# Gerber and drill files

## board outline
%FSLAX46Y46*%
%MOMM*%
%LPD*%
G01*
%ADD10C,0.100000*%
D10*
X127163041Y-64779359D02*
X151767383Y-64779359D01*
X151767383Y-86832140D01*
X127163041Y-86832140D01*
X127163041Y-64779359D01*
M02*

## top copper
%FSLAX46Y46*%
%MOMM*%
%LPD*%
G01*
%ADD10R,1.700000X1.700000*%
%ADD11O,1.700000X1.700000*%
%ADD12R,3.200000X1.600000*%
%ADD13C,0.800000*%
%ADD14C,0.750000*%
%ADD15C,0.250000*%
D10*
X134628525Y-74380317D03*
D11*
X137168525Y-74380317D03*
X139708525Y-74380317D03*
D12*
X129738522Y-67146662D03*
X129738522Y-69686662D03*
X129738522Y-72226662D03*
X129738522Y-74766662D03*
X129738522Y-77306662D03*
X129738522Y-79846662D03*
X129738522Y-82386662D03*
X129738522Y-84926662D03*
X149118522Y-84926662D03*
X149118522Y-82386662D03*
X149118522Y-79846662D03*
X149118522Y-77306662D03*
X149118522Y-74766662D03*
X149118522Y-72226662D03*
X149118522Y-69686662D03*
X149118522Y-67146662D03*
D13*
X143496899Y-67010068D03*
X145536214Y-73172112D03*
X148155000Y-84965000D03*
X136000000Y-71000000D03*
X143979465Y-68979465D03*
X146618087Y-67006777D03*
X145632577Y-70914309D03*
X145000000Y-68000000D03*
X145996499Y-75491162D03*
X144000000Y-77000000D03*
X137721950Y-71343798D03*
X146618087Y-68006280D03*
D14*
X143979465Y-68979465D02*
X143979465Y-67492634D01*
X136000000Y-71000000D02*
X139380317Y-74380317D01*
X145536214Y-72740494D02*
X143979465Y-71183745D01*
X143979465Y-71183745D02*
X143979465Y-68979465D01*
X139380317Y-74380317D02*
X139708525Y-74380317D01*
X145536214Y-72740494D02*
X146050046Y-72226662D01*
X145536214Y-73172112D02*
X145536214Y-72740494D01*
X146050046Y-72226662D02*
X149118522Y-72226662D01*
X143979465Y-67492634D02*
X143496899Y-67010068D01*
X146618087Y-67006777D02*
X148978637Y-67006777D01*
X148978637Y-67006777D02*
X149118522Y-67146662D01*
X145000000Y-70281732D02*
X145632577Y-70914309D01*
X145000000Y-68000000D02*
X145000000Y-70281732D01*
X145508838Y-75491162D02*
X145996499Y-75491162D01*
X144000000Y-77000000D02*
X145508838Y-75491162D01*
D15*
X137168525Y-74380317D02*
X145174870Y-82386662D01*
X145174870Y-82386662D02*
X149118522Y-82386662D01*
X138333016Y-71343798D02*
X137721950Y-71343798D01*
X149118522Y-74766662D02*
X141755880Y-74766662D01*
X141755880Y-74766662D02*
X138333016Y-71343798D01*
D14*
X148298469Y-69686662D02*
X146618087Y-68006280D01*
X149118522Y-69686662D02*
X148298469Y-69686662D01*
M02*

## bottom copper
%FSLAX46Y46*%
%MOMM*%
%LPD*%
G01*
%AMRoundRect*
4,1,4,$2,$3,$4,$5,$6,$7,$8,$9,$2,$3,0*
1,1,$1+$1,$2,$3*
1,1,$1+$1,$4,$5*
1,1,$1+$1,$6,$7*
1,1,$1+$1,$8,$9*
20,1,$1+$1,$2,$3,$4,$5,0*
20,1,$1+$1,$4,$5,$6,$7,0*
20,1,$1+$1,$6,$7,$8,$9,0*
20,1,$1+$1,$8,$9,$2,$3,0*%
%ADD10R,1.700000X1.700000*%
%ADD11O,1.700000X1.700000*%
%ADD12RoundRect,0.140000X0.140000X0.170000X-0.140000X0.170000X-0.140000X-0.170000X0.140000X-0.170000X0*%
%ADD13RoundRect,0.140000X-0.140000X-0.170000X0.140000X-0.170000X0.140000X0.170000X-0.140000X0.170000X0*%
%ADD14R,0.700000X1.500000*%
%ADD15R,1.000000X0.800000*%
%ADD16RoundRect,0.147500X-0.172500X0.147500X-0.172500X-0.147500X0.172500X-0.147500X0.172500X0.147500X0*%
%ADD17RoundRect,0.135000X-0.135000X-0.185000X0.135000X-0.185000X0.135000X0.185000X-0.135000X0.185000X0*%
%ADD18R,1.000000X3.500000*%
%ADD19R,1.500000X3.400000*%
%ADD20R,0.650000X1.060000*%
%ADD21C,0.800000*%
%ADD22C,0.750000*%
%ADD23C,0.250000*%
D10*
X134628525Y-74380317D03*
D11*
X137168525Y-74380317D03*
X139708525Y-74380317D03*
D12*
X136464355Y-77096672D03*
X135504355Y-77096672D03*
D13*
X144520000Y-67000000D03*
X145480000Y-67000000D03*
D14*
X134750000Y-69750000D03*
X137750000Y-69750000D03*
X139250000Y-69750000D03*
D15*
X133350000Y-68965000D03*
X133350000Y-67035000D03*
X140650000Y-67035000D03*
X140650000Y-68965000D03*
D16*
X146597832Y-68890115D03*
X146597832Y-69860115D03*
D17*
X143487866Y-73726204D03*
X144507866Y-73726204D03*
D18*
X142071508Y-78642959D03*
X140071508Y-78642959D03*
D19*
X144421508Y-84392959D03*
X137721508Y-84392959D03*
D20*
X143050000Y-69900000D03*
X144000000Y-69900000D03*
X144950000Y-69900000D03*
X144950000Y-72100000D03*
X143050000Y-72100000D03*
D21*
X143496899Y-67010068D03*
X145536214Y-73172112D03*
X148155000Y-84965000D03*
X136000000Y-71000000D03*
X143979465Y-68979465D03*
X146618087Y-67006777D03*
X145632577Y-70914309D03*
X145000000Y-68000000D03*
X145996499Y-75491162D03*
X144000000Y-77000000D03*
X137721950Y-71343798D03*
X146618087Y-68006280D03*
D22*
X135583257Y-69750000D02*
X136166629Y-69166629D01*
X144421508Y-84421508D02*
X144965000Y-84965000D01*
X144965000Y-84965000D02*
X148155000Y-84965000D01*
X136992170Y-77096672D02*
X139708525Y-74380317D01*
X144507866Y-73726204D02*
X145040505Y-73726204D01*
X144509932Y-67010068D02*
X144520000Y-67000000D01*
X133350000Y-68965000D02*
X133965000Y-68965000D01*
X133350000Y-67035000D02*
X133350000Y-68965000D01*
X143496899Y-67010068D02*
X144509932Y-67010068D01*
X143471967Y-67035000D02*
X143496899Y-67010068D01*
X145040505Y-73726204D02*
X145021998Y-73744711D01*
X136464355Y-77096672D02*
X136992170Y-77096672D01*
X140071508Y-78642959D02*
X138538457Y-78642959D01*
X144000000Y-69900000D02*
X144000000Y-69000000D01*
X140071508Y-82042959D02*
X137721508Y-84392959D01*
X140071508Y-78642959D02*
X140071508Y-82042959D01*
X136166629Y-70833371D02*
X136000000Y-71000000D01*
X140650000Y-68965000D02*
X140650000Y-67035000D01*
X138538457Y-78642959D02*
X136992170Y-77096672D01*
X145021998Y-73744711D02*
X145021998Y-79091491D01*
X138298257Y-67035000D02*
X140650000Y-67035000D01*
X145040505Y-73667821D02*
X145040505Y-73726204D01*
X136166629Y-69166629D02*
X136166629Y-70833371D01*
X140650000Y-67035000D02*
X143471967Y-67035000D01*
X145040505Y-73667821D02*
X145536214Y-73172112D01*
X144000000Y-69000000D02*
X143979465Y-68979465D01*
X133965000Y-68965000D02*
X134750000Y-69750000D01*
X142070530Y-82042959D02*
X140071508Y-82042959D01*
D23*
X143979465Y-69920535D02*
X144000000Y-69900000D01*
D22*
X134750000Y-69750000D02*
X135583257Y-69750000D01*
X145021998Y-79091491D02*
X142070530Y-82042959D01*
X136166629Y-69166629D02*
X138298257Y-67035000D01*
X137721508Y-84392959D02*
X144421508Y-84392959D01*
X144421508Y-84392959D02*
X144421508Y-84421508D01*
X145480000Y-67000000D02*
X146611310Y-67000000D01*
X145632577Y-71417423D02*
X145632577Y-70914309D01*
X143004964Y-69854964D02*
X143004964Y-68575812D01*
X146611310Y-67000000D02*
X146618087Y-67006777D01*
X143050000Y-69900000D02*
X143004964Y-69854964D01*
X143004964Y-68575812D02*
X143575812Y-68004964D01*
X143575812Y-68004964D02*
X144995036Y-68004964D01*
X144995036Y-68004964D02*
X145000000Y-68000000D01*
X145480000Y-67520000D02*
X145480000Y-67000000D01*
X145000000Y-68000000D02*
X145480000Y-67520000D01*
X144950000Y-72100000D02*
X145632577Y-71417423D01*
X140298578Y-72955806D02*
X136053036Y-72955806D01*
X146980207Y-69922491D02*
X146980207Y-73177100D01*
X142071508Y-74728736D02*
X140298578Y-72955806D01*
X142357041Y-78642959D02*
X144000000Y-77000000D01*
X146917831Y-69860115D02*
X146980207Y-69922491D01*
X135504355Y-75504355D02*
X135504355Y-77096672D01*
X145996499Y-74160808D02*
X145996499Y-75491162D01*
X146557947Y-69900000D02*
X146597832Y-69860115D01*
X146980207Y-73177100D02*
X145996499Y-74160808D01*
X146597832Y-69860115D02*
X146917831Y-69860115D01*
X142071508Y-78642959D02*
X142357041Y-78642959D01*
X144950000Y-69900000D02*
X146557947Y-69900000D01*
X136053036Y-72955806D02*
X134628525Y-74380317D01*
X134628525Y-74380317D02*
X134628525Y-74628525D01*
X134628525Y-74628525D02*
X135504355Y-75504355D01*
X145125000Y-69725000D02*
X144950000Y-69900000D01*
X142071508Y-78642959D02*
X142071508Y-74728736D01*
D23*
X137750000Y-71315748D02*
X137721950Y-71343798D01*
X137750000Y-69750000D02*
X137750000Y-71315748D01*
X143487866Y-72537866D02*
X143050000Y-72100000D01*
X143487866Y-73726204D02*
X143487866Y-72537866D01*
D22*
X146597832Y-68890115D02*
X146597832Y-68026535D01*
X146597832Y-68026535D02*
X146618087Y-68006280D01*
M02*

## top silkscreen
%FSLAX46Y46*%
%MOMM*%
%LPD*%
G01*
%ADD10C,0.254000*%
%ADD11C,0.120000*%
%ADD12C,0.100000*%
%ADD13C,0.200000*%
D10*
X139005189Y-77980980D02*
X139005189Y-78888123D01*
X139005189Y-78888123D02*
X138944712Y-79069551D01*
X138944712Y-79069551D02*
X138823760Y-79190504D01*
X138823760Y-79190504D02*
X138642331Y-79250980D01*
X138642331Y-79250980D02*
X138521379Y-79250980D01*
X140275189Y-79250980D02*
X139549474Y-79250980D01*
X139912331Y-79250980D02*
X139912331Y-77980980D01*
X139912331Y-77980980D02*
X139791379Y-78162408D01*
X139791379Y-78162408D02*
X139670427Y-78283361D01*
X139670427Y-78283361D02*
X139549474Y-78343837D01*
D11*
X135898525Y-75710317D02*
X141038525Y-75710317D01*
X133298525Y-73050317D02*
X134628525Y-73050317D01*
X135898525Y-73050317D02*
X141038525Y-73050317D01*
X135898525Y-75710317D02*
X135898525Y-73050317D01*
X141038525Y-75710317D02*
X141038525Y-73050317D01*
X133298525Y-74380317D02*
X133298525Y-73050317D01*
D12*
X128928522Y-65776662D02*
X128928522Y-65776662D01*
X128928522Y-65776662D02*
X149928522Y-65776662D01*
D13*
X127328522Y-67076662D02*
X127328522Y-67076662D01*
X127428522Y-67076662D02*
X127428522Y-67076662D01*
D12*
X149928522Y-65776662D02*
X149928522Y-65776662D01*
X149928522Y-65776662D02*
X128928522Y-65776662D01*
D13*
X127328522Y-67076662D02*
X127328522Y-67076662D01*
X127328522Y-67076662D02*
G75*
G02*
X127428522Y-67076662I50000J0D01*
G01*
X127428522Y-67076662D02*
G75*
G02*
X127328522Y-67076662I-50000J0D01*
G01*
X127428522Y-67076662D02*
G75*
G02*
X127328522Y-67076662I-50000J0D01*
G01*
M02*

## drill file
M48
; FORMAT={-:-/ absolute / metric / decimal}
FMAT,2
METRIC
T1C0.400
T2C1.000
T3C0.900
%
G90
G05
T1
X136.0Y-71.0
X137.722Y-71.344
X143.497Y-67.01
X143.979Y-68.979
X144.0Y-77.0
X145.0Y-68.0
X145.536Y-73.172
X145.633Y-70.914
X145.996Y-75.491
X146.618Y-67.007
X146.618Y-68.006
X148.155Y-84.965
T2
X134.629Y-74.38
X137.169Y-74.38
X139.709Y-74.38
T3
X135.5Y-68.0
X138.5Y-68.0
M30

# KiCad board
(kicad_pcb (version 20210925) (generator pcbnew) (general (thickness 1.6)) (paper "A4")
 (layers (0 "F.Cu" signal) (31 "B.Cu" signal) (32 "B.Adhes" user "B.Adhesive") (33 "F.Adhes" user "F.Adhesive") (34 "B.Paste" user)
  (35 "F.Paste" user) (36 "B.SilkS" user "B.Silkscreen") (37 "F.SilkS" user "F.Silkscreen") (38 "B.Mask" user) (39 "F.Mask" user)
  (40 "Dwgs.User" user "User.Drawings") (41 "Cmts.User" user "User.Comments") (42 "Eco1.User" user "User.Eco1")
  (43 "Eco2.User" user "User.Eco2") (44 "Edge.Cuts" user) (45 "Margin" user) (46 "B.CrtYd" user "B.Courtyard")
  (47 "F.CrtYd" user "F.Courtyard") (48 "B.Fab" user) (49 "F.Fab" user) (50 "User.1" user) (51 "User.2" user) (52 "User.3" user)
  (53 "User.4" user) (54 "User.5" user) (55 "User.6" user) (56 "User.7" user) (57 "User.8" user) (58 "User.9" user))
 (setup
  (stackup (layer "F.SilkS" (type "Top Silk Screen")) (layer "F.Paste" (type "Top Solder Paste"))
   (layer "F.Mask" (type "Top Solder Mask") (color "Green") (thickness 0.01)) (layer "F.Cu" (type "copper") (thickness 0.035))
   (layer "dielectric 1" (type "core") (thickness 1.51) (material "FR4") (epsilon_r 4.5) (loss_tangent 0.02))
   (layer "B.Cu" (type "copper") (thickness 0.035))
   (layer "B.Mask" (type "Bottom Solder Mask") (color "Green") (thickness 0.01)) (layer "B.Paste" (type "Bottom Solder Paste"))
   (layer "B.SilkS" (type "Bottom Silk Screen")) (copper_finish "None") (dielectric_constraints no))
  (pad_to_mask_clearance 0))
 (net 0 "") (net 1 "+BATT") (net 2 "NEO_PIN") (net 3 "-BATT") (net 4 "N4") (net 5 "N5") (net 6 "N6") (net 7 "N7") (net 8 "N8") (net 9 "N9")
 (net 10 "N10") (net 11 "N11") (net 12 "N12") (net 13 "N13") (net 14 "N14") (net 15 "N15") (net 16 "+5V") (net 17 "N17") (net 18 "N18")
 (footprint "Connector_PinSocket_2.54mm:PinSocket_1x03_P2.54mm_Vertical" (layer "F.Cu") (at 134.628525 74.380317 90)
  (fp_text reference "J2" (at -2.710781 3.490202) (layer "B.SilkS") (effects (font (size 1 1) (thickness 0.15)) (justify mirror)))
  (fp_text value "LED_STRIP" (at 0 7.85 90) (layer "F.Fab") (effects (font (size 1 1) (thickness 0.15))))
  (fp_line (start -1.33 1.27) (end -1.33 6.41) (layer "F.SilkS") (width 0.12))
  (fp_line (start 1.33 -1.33) (end 1.33 0) (layer "F.SilkS") (width 0.12))
  (fp_line (start 1.33 1.27) (end 1.33 6.41) (layer "F.SilkS") (width 0.12))
  (fp_line (start -1.33 1.27) (end 1.33 1.27) (layer "F.SilkS") (width 0.12))
  (fp_line (start -1.33 6.41) (end 1.33 6.41) (layer "F.SilkS") (width 0.12))
  (fp_line (start 0 -1.33) (end 1.33 -1.33) (layer "F.SilkS") (width 0.12))
  (pad "1" thru_hole rect locked (at 0 0 90) (size 1.7 1.7) (drill 1) (layers *.Cu *.Mask) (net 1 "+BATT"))
  (pad "2" thru_hole oval locked (at 0 2.54 90) (size 1.7 1.7) (drill 1) (layers *.Cu *.Mask) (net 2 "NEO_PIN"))
  (pad "3" thru_hole oval locked (at 0 5.08 90) (size 1.7 1.7) (drill 1) (layers *.Cu *.Mask) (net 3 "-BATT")))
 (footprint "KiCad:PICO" (layer "F.Cu") (at 128.928522 116.776662)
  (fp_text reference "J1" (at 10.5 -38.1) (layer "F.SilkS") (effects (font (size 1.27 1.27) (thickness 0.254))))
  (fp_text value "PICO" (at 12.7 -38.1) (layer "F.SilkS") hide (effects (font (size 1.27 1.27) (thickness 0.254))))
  (fp_line (start 0 -51) (end 0 -51) (layer "F.SilkS") (width 0.1))
  (fp_line (start 0 -51) (end 21 -51) (layer "F.SilkS") (width 0.1))
  (fp_line (start -1.6 -49.7) (end -1.6 -49.7) (layer "F.SilkS") (width 0.2))
  (fp_line (start -1.5 -49.7) (end -1.5 -49.7) (layer "F.SilkS") (width 0.2))
  (fp_line (start 21 -51) (end 21 -51) (layer "F.SilkS") (width 0.1))
  (fp_line (start 21 -51) (end 0 -51) (layer "F.SilkS") (width 0.1))
  (fp_line (start -1.6 -49.7) (end -1.6 -49.7) (layer "F.SilkS") (width 0.2))
  (fp_arc (start -1.55 -49.7) (end -1.5 -49.7) (angle -180) (layer "F.SilkS") (width 0.2))
  (fp_arc (start -1.55 -49.7) (end -1.6 -49.7) (angle -180) (layer "F.SilkS") (width 0.2))
  (fp_arc (start -1.55 -49.7) (end -1.6 -49.7) (angle -180) (layer "F.SilkS") (width 0.2))
  (pad "1" smd rect (at 0.81 -49.63 90) (size 1.6 3.2) (layers "F.Cu" "F.Paste" "F.Mask") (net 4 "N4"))
  (pad "2" smd rect (at 0.81 -47.09 90) (size 1.6 3.2) (layers "F.Cu" "F.Paste" "F.Mask") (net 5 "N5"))
  (pad "3" smd rect (at 0.81 -44.55 90) (size 1.6 3.2) (layers "F.Cu" "F.Paste" "F.Mask") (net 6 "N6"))
  (pad "4" smd rect (at 0.81 -42.01 90) (size 1.6 3.2) (layers "F.Cu" "F.Paste" "F.Mask") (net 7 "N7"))
  (pad "5" smd rect (at 0.81 -39.47 90) (size 1.6 3.2) (layers "F.Cu" "F.Paste" "F.Mask") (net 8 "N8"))
  (pad "6" smd rect (at 0.81 -36.93 90) (size 1.6 3.2) (layers "F.Cu" "F.Paste" "F.Mask") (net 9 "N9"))
  (pad "7" smd rect (at 0.81 -34.39 90) (size 1.6 3.2) (layers "F.Cu" "F.Paste" "F.Mask") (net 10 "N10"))
  (pad "8" smd rect (at 0.81 -31.85 90) (size 1.6 3.2) (layers "F.Cu" "F.Paste" "F.Mask") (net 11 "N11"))
  (pad "33" smd rect (at 20.19 -31.85 90) (size 1.6 3.2) (layers "F.Cu" "F.Paste" "F.Mask") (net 3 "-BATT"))
  (pad "34" smd rect (at 20.19 -34.39 90) (size 1.6 3.2) (layers "F.Cu" "F.Paste" "F.Mask") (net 2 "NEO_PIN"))
  (pad "35" smd rect (at 20.19 -36.93 90) (size 1.6 3.2) (layers "F.Cu" "F.Paste" "F.Mask") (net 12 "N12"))
  (pad "36" smd rect (at 20.19 -39.47 90) (size 1.6 3.2) (layers "F.Cu" "F.Paste" "F.Mask") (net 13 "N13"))
  (pad "37" smd rect (at 20.19 -42.01 90) (size 1.6 3.2) (layers "F.Cu" "F.Paste" "F.Mask") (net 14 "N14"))
  (pad "38" smd rect (at 20.19 -44.55 90) (size 1.6 3.2) (layers "F.Cu" "F.Paste" "F.Mask") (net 3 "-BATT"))
  (pad "39" smd rect (at 20.19 -47.09 90) (size 1.6 3.2) (layers "F.Cu" "F.Paste" "F.Mask") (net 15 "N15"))
  (pad "40" smd rect (at 20.19 -49.63 90) (size 1.6 3.2) (layers "F.Cu" "F.Paste" "F.Mask") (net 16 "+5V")))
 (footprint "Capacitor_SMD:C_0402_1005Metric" (layer "B.Cu") (at 135.984355 77.096672 180)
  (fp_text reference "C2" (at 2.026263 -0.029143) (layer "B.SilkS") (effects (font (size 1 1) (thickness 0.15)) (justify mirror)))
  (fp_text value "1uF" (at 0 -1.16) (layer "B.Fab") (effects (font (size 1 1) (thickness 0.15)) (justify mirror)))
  (pad "1" smd roundrect locked (at -0.48 0 180) (size 0.56 0.62) (layers "B.Cu" "B.Paste" "B.Mask") (roundrect_rratio 0.25) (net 3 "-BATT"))
  (pad "2" smd roundrect locked (at 0.48 0 180) (size 0.56 0.62) (layers "B.Cu" "B.Paste" "B.Mask") (roundrect_rratio 0.25) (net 1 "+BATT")))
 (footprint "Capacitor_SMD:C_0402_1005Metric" (layer "B.Cu") (at 145 67)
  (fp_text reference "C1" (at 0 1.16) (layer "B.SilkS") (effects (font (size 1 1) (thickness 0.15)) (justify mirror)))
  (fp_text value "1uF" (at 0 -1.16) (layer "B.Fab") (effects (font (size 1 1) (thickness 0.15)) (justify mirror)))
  (pad "1" smd roundrect locked (at -0.48 0) (size 0.56 0.62) (layers "B.Cu" "B.Paste" "B.Mask") (roundrect_rratio 0.25) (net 3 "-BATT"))
  (pad "2" smd roundrect locked (at 0.48 0) (size 0.56 0.62) (layers "B.Cu" "B.Paste" "B.Mask") (roundrect_rratio 0.25) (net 16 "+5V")))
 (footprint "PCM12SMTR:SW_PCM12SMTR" (layer "B.Cu") (at 137 68)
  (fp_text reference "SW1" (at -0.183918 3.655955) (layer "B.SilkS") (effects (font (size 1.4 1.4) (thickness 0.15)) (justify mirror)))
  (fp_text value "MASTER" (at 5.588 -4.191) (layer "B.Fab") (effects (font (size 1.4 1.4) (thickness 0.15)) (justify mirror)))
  (pad "" np_thru_hole circle locked (at -1.5 0) (size 0.9 0.9) (drill 0.9) (layers *.Cu *.Mask))
  (pad "" np_thru_hole circle locked (at 1.5 0) (size 0.9 0.9) (drill 0.9) (layers *.Cu *.Mask))
  (pad "1" smd rect locked (at -2.25 1.75) (size 0.7 1.5) (layers "B.Cu" "B.Paste" "B.Mask") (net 3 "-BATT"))
  (pad "2" smd rect locked (at 0.75 1.75) (size 0.7 1.5) (layers "B.Cu" "B.Paste" "B.Mask") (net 14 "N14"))
  (pad "3" smd rect locked (at 2.25 1.75) (size 0.7 1.5) (layers "B.Cu" "B.Paste" "B.Mask") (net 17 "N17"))
  (pad "S1" smd rect locked (at -3.65 0.965) (size 1 0.8) (layers "B.Cu" "B.Paste" "B.Mask") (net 3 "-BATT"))
  (pad "S2" smd rect locked (at -3.65 -0.965) (size 1 0.8) (layers "B.Cu" "B.Paste" "B.Mask") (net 3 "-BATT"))
  (pad "S3" smd rect locked (at 3.65 -0.965) (size 1 0.8) (layers "B.Cu" "B.Paste" "B.Mask") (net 3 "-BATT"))
  (pad "S4" smd rect locked (at 3.65 0.965) (size 1 0.8) (layers "B.Cu" "B.Paste" "B.Mask") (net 3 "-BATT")))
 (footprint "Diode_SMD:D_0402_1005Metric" (layer "B.Cu") (at 146.597832 69.375115 -90)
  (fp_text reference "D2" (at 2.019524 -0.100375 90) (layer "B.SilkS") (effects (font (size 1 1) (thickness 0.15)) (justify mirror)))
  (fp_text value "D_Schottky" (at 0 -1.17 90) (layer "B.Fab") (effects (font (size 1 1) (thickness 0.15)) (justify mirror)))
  (pad "1" smd roundrect locked (at -0.485 0 270) (size 0.59 0.64) (layers "B.Cu" "B.Paste" "B.Mask") (roundrect_rratio 0.25) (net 15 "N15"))
  (pad "2" smd roundrect locked (at 0.485 0 270) (size 0.59 0.64) (layers "B.Cu" "B.Paste" "B.Mask") (roundrect_rratio 0.25) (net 1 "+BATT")))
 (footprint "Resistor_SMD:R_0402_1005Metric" (layer "B.Cu") (at 143.997866 73.726204)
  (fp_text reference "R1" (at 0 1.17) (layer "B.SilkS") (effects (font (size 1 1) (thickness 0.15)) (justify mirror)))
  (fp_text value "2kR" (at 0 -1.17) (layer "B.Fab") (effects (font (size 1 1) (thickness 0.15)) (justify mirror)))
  (pad "1" smd roundrect locked (at -0.51 0) (size 0.54 0.64) (layers "B.Cu" "B.Paste" "B.Mask") (roundrect_rratio 0.25) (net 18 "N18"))
  (pad "2" smd roundrect locked (at 0.51 0) (size 0.54 0.64) (layers "B.Cu" "B.Paste" "B.Mask") (roundrect_rratio 0.25) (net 3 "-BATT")))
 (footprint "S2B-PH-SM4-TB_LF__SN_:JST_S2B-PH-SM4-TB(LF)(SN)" (layer "B.Cu") (at 141.071508 78.642959 180)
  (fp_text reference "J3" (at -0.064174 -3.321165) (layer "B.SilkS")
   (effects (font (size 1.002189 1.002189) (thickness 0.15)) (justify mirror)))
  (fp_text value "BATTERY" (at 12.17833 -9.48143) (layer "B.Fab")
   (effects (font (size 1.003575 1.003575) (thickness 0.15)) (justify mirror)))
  (pad "1" smd rect locked (at -1 0 180) (size 1 3.5) (layers "B.Cu" "B.Paste" "B.Mask") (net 1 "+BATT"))
  (pad "2" smd rect locked (at 1 0 180) (size 1 3.5) (layers "B.Cu" "B.Paste" "B.Mask") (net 3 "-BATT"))
  (pad "S1" smd rect locked (at -3.35 -5.75 180) (size 1.5 3.4) (layers "B.Cu" "B.Paste" "B.Mask") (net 3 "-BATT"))
  (pad "S2" smd rect locked (at 3.35 -5.75 180) (size 1.5 3.4) (layers "B.Cu" "B.Paste" "B.Mask") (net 3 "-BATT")))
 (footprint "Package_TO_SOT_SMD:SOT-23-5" (layer "B.Cu") (at 144 71 -90)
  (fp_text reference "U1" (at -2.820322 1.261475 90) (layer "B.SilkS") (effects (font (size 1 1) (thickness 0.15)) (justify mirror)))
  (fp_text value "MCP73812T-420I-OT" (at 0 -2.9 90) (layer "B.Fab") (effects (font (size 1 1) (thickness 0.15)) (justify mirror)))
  (pad "1" smd rect locked (at -1.1 0.95 270) (size 1.06 0.65) (layers "B.Cu" "B.Paste" "B.Mask") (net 16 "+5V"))
  (pad "2" smd rect locked (at -1.1 0 270) (size 1.06 0.65) (layers "B.Cu" "B.Paste" "B.Mask") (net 3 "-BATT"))
  (pad "3" smd rect locked (at -1.1 -0.95 270) (size 1.06 0.65) (layers "B.Cu" "B.Paste" "B.Mask") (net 1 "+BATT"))
  (pad "4" smd rect locked (at 1.1 -0.95 270) (size 1.06 0.65) (layers "B.Cu" "B.Paste" "B.Mask") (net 16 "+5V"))
  (pad "5" smd rect locked (at 1.1 0.95 270) (size 1.06 0.65) (layers "B.Cu" "B.Paste" "B.Mask") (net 18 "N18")))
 (gr_rect (start 151.767383 86.83214) (end 127.163041 64.779359) (layer "Edge.Cuts") (width 0.1) (fill none))
 (segment (start 143.979465 68.979465) (end 143.979465 67.492634) (width 0.75) (layer "F.Cu") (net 3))
 (segment (start 136 71) (end 139.380317 74.380317) (width 0.75) (layer "F.Cu") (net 3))
 (segment (start 145.536214 72.740494) (end 143.979465 71.183745) (width 0.75) (layer "F.Cu") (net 3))
 (segment (start 143.979465 71.183745) (end 143.979465 68.979465) (width 0.75) (layer "F.Cu") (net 3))
 (segment (start 139.380317 74.380317) (end 139.708525 74.380317) (width 0.75) (layer "F.Cu") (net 3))
 (segment (start 145.536214 72.740494) (end 146.050046 72.226662) (width 0.75) (layer "F.Cu") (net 3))
 (segment (start 145.536214 73.172112) (end 145.536214 72.740494) (width 0.75) (layer "F.Cu") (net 3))
 (segment (start 146.050046 72.226662) (end 149.118522 72.226662) (width 0.75) (layer "F.Cu") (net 3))
 (segment (start 143.979465 67.492634) (end 143.496899 67.010068) (width 0.75) (layer "F.Cu") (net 3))
 (via (at 143.496899 67.010068) (size 0.8) (drill 0.4) (layers "F.Cu" "B.Cu") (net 3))
 (via (at 145.536214 73.172112) (size 0.8) (drill 0.4) (layers "F.Cu" "B.Cu") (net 3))
 (via (at 148.155 84.965) (size 0.8) (drill 0.4) (layers "F.Cu" "B.Cu") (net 3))
 (via (at 136 71) (size 0.8) (drill 0.4) (layers "F.Cu" "B.Cu") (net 3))
 (via (at 143.979465 68.979465) (size 0.8) (drill 0.4) (layers "F.Cu" "B.Cu") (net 3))
 (segment (start 135.583257 69.75) (end 136.166629 69.166629) (width 0.75) (layer "B.Cu") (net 3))
 (segment (start 144.421508 84.421508) (end 144.965 84.965) (width 0.75) (layer "B.Cu") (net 3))
 (segment (start 144.965 84.965) (end 148.155 84.965) (width 0.75) (layer "B.Cu") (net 3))
 (segment (start 136.99217 77.096672) (end 139.708525 74.380317) (width 0.75) (layer "B.Cu") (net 3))
 (segment (start 144.507866 73.726204) (end 145.040505 73.726204) (width 0.75) (layer "B.Cu") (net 3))
 (segment (start 144.509932 67.010068) (end 144.52 67) (width 0.75) (layer "B.Cu") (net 3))
 (segment (start 133.35 68.965) (end 133.965 68.965) (width 0.75) (layer "B.Cu") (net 3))
 (segment (start 133.35 67.035) (end 133.35 68.965) (width 0.75) (layer "B.Cu") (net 3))
 (segment (start 143.496899 67.010068) (end 144.509932 67.010068) (width 0.75) (layer "B.Cu") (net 3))
 (segment (start 143.471967 67.035) (end 143.496899 67.010068) (width 0.75) (layer "B.Cu") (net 3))
 (segment (start 145.040505 73.726204) (end 145.021998 73.744711) (width 0.75) (layer "B.Cu") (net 3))
 (segment (start 136.464355 77.096672) (end 136.99217 77.096672) (width 0.75) (layer "B.Cu") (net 3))
 (segment (start 140.071508 78.642959) (end 138.538457 78.642959) (width 0.75) (layer "B.Cu") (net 3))
 (segment (start 144 69.9) (end 144 69) (width 0.75) (layer "B.Cu") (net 3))
 (segment (start 140.071508 82.042959) (end 137.721508 84.392959) (width 0.75) (layer "B.Cu") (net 3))
 (segment (start 140.071508 78.642959) (end 140.071508 82.042959) (width 0.75) (layer "B.Cu") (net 3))
 (segment (start 136.166629 70.833371) (end 136 71) (width 0.75) (layer "B.Cu") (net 3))
 (segment (start 140.65 68.965) (end 140.65 67.035) (width 0.75) (layer "B.Cu") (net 3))
 (segment (start 138.538457 78.642959) (end 136.99217 77.096672) (width 0.75) (layer "B.Cu") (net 3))
 (segment (start 145.021998 73.744711) (end 145.021998 79.091491) (width 0.75) (layer "B.Cu") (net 3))
 (segment (start 138.298257 67.035) (end 140.65 67.035) (width 0.75) (layer "B.Cu") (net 3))
 (segment (start 145.040505 73.667821) (end 145.040505 73.726204) (width 0.75) (layer "B.Cu") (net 3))
 (segment (start 136.166629 69.166629) (end 136.166629 70.833371) (width 0.75) (layer "B.Cu") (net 3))
 (segment (start 140.65 67.035) (end 143.471967 67.035) (width 0.75) (layer "B.Cu") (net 3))
 (segment (start 145.040505 73.667821) (end 145.536214 73.172112) (width 0.75) (layer "B.Cu") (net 3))
 (segment (start 144 69) (end 143.979465 68.979465) (width 0.75) (layer "B.Cu") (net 3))
 (segment (start 133.965 68.965) (end 134.75 69.75) (width 0.75) (layer "B.Cu") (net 3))
 (segment (start 142.07053 82.042959) (end 140.071508 82.042959) (width 0.75) (layer "B.Cu") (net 3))
 (segment (start 143.979465 69.920535) (end 144 69.9) (width 0.25) (layer "B.Cu") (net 3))
 (segment (start 134.75 69.75) (end 135.583257 69.75) (width 0.75) (layer "B.Cu") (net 3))
 (segment (start 145.021998 79.091491) (end 142.07053 82.042959) (width 0.75) (layer "B.Cu") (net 3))
 (segment (start 136.166629 69.166629) (end 138.298257 67.035) (width 0.75) (layer "B.Cu") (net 3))
 (segment (start 137.721508 84.392959) (end 144.421508 84.392959) (width 0.75) (layer "B.Cu") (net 3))
 (segment (start 144.421508 84.392959) (end 144.421508 84.421508) (width 0.75) (layer "B.Cu") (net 3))
 (segment (start 146.618087 67.006777) (end 148.978637 67.006777) (width 0.75) (layer "F.Cu") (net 16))
 (segment (start 148.978637 67.006777) (end 149.118522 67.146662) (width 0.75) (layer "F.Cu") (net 16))
 (segment (start 145 70.281732) (end 145.632577 70.914309) (width 0.75) (layer "F.Cu") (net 16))
 (segment (start 145 68) (end 145 70.281732) (width 0.75) (layer "F.Cu") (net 16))
 (via (at 146.618087 67.006777) (size 0.8) (drill 0.4) (layers "F.Cu" "B.Cu") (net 16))
 (via (at 145.632577 70.914309) (size 0.8) (drill 0.4) (layers "F.Cu" "B.Cu") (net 16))
 (via (at 145 68) (size 0.8) (drill 0.4) (layers "F.Cu" "B.Cu") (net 16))
 (segment (start 145.48 67) (end 146.61131 67) (width 0.75) (layer "B.Cu") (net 16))
 (segment (start 145.632577 71.417423) (end 145.632577 70.914309) (width 0.75) (layer "B.Cu") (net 16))
 (segment (start 143.004964 69.854964) (end 143.004964 68.575812) (width 0.75) (layer "B.Cu") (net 16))
 (segment (start 146.61131 67) (end 146.618087 67.006777) (width 0.75) (layer "B.Cu") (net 16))
 (segment (start 143.05 69.9) (end 143.004964 69.854964) (width 0.75) (layer "B.Cu") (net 16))
 (segment (start 143.004964 68.575812) (end 143.575812 68.004964) (width 0.75) (layer "B.Cu") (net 16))
 (segment (start 143.575812 68.004964) (end 144.995036 68.004964) (width 0.75) (layer "B.Cu") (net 16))
 (segment (start 144.995036 68.004964) (end 145 68) (width 0.75) (layer "B.Cu") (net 16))
 (segment (start 145.48 67.52) (end 145.48 67) (width 0.75) (layer "B.Cu") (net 16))
 (segment (start 145 68) (end 145.48 67.52) (width 0.75) (layer "B.Cu") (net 16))
 (segment (start 144.95 72.1) (end 145.632577 71.417423) (width 0.75) (layer "B.Cu") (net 16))
 (segment (start 145.508838 75.491162) (end 145.996499 75.491162) (width 0.75) (layer "F.Cu") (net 1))
 (segment (start 144 77) (end 145.508838 75.491162) (width 0.75) (layer "F.Cu") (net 1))
 (via (at 145.996499 75.491162) (size 0.8) (drill 0.4) (layers "F.Cu" "B.Cu") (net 1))
 (via (at 144 77) (size 0.8) (drill 0.4) (layers "F.Cu" "B.Cu") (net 1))
 (segment (start 140.298578 72.955806) (end 136.053036 72.955806) (width 0.75) (layer "B.Cu") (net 1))
 (segment (start 146.980207 69.922491) (end 146.980207 73.1771) (width 0.75) (layer "B.Cu") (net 1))
 (segment (start 142.071508 74.728736) (end 140.298578 72.955806) (width 0.75) (layer "B.Cu") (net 1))
 (segment (start 142.357041 78.642959) (end 144 77) (width 0.75) (layer "B.Cu") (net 1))
 (segment (start 146.917831 69.860115) (end 146.980207 69.922491) (width 0.75) (layer "B.Cu") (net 1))
 (segment (start 135.504355 75.504355) (end 135.504355 77.096672) (width 0.75) (layer "B.Cu") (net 1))
 (segment (start 145.996499 74.160808) (end 145.996499 75.491162) (width 0.75) (layer "B.Cu") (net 1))
 (segment (start 146.557947 69.9) (end 146.597832 69.860115) (width 0.75) (layer "B.Cu") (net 1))
 (segment (start 146.980207 73.1771) (end 145.996499 74.160808) (width 0.75) (layer "B.Cu") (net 1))
 (segment (start 146.597832 69.860115) (end 146.917831 69.860115) (width 0.75) (layer "B.Cu") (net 1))
 (segment (start 142.071508 78.642959) (end 142.357041 78.642959) (width 0.75) (layer "B.Cu") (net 1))
 (segment (start 144.95 69.9) (end 146.557947 69.9) (width 0.75) (layer "B.Cu") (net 1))
 (segment (start 136.053036 72.955806) (end 134.628525 74.380317) (width 0.75) (layer "B.Cu") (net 1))
 (segment (start 134.628525 74.380317) (end 134.628525 74.628525) (width 0.75) (layer "B.Cu") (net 1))
 (segment (start 134.628525 74.628525) (end 135.504355 75.504355) (width 0.75) (layer "B.Cu") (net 1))
 (segment (start 145.125 69.725) (end 144.95 69.9) (width 0.75) (layer "B.Cu") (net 1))
 (segment (start 142.071508 78.642959) (end 142.071508 74.728736) (width 0.75) (layer "B.Cu") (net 1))
 (segment (start 137.168525 74.380317) (end 145.17487 82.386662) (width 0.25) (layer "F.Cu") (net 2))
 (segment (start 145.17487 82.386662) (end 149.118522 82.386662) (width 0.25) (layer "F.Cu") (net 2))
 (segment (start 138.333016 71.343798) (end 137.72195 71.343798) (width 0.25) (layer "F.Cu") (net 14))
 (segment (start 149.118522 74.766662) (end 141.75588 74.766662) (width 0.25) (layer "F.Cu") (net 14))
 (segment (start 141.75588 74.766662) (end 138.333016 71.343798) (width 0.25) (layer "F.Cu") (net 14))
 (via (at 137.72195 71.343798) (size 0.8) (drill 0.4) (layers "F.Cu" "B.Cu") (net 14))
 (segment (start 137.75 71.315748) (end 137.72195 71.343798) (width 0.25) (layer "B.Cu") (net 14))
 (segment (start 137.75 69.75) (end 137.75 71.315748) (width 0.25) (layer "B.Cu") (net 14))
 (segment (start 143.487866 72.537866) (end 143.05 72.1) (width 0.25) (layer "B.Cu") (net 18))
 (segment (start 143.487866 73.726204) (end 143.487866 72.537866) (width 0.25) (layer "B.Cu") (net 18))
 (segment (start 148.298469 69.686662) (end 146.618087 68.00628) (width 0.75) (layer "F.Cu") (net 15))
 (segment (start 149.118522 69.686662) (end 148.298469 69.686662) (width 0.75) (layer "F.Cu") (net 15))
 (via (at 146.618087 68.00628) (size 0.8) (drill 0.4) (layers "F.Cu" "B.Cu") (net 15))
 (segment (start 146.597832 68.890115) (end 146.597832 68.026535) (width 0.75) (layer "B.Cu") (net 15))
 (segment (start 146.597832 68.026535) (end 146.618087 68.00628) (width 0.75) (layer "B.Cu") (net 15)))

